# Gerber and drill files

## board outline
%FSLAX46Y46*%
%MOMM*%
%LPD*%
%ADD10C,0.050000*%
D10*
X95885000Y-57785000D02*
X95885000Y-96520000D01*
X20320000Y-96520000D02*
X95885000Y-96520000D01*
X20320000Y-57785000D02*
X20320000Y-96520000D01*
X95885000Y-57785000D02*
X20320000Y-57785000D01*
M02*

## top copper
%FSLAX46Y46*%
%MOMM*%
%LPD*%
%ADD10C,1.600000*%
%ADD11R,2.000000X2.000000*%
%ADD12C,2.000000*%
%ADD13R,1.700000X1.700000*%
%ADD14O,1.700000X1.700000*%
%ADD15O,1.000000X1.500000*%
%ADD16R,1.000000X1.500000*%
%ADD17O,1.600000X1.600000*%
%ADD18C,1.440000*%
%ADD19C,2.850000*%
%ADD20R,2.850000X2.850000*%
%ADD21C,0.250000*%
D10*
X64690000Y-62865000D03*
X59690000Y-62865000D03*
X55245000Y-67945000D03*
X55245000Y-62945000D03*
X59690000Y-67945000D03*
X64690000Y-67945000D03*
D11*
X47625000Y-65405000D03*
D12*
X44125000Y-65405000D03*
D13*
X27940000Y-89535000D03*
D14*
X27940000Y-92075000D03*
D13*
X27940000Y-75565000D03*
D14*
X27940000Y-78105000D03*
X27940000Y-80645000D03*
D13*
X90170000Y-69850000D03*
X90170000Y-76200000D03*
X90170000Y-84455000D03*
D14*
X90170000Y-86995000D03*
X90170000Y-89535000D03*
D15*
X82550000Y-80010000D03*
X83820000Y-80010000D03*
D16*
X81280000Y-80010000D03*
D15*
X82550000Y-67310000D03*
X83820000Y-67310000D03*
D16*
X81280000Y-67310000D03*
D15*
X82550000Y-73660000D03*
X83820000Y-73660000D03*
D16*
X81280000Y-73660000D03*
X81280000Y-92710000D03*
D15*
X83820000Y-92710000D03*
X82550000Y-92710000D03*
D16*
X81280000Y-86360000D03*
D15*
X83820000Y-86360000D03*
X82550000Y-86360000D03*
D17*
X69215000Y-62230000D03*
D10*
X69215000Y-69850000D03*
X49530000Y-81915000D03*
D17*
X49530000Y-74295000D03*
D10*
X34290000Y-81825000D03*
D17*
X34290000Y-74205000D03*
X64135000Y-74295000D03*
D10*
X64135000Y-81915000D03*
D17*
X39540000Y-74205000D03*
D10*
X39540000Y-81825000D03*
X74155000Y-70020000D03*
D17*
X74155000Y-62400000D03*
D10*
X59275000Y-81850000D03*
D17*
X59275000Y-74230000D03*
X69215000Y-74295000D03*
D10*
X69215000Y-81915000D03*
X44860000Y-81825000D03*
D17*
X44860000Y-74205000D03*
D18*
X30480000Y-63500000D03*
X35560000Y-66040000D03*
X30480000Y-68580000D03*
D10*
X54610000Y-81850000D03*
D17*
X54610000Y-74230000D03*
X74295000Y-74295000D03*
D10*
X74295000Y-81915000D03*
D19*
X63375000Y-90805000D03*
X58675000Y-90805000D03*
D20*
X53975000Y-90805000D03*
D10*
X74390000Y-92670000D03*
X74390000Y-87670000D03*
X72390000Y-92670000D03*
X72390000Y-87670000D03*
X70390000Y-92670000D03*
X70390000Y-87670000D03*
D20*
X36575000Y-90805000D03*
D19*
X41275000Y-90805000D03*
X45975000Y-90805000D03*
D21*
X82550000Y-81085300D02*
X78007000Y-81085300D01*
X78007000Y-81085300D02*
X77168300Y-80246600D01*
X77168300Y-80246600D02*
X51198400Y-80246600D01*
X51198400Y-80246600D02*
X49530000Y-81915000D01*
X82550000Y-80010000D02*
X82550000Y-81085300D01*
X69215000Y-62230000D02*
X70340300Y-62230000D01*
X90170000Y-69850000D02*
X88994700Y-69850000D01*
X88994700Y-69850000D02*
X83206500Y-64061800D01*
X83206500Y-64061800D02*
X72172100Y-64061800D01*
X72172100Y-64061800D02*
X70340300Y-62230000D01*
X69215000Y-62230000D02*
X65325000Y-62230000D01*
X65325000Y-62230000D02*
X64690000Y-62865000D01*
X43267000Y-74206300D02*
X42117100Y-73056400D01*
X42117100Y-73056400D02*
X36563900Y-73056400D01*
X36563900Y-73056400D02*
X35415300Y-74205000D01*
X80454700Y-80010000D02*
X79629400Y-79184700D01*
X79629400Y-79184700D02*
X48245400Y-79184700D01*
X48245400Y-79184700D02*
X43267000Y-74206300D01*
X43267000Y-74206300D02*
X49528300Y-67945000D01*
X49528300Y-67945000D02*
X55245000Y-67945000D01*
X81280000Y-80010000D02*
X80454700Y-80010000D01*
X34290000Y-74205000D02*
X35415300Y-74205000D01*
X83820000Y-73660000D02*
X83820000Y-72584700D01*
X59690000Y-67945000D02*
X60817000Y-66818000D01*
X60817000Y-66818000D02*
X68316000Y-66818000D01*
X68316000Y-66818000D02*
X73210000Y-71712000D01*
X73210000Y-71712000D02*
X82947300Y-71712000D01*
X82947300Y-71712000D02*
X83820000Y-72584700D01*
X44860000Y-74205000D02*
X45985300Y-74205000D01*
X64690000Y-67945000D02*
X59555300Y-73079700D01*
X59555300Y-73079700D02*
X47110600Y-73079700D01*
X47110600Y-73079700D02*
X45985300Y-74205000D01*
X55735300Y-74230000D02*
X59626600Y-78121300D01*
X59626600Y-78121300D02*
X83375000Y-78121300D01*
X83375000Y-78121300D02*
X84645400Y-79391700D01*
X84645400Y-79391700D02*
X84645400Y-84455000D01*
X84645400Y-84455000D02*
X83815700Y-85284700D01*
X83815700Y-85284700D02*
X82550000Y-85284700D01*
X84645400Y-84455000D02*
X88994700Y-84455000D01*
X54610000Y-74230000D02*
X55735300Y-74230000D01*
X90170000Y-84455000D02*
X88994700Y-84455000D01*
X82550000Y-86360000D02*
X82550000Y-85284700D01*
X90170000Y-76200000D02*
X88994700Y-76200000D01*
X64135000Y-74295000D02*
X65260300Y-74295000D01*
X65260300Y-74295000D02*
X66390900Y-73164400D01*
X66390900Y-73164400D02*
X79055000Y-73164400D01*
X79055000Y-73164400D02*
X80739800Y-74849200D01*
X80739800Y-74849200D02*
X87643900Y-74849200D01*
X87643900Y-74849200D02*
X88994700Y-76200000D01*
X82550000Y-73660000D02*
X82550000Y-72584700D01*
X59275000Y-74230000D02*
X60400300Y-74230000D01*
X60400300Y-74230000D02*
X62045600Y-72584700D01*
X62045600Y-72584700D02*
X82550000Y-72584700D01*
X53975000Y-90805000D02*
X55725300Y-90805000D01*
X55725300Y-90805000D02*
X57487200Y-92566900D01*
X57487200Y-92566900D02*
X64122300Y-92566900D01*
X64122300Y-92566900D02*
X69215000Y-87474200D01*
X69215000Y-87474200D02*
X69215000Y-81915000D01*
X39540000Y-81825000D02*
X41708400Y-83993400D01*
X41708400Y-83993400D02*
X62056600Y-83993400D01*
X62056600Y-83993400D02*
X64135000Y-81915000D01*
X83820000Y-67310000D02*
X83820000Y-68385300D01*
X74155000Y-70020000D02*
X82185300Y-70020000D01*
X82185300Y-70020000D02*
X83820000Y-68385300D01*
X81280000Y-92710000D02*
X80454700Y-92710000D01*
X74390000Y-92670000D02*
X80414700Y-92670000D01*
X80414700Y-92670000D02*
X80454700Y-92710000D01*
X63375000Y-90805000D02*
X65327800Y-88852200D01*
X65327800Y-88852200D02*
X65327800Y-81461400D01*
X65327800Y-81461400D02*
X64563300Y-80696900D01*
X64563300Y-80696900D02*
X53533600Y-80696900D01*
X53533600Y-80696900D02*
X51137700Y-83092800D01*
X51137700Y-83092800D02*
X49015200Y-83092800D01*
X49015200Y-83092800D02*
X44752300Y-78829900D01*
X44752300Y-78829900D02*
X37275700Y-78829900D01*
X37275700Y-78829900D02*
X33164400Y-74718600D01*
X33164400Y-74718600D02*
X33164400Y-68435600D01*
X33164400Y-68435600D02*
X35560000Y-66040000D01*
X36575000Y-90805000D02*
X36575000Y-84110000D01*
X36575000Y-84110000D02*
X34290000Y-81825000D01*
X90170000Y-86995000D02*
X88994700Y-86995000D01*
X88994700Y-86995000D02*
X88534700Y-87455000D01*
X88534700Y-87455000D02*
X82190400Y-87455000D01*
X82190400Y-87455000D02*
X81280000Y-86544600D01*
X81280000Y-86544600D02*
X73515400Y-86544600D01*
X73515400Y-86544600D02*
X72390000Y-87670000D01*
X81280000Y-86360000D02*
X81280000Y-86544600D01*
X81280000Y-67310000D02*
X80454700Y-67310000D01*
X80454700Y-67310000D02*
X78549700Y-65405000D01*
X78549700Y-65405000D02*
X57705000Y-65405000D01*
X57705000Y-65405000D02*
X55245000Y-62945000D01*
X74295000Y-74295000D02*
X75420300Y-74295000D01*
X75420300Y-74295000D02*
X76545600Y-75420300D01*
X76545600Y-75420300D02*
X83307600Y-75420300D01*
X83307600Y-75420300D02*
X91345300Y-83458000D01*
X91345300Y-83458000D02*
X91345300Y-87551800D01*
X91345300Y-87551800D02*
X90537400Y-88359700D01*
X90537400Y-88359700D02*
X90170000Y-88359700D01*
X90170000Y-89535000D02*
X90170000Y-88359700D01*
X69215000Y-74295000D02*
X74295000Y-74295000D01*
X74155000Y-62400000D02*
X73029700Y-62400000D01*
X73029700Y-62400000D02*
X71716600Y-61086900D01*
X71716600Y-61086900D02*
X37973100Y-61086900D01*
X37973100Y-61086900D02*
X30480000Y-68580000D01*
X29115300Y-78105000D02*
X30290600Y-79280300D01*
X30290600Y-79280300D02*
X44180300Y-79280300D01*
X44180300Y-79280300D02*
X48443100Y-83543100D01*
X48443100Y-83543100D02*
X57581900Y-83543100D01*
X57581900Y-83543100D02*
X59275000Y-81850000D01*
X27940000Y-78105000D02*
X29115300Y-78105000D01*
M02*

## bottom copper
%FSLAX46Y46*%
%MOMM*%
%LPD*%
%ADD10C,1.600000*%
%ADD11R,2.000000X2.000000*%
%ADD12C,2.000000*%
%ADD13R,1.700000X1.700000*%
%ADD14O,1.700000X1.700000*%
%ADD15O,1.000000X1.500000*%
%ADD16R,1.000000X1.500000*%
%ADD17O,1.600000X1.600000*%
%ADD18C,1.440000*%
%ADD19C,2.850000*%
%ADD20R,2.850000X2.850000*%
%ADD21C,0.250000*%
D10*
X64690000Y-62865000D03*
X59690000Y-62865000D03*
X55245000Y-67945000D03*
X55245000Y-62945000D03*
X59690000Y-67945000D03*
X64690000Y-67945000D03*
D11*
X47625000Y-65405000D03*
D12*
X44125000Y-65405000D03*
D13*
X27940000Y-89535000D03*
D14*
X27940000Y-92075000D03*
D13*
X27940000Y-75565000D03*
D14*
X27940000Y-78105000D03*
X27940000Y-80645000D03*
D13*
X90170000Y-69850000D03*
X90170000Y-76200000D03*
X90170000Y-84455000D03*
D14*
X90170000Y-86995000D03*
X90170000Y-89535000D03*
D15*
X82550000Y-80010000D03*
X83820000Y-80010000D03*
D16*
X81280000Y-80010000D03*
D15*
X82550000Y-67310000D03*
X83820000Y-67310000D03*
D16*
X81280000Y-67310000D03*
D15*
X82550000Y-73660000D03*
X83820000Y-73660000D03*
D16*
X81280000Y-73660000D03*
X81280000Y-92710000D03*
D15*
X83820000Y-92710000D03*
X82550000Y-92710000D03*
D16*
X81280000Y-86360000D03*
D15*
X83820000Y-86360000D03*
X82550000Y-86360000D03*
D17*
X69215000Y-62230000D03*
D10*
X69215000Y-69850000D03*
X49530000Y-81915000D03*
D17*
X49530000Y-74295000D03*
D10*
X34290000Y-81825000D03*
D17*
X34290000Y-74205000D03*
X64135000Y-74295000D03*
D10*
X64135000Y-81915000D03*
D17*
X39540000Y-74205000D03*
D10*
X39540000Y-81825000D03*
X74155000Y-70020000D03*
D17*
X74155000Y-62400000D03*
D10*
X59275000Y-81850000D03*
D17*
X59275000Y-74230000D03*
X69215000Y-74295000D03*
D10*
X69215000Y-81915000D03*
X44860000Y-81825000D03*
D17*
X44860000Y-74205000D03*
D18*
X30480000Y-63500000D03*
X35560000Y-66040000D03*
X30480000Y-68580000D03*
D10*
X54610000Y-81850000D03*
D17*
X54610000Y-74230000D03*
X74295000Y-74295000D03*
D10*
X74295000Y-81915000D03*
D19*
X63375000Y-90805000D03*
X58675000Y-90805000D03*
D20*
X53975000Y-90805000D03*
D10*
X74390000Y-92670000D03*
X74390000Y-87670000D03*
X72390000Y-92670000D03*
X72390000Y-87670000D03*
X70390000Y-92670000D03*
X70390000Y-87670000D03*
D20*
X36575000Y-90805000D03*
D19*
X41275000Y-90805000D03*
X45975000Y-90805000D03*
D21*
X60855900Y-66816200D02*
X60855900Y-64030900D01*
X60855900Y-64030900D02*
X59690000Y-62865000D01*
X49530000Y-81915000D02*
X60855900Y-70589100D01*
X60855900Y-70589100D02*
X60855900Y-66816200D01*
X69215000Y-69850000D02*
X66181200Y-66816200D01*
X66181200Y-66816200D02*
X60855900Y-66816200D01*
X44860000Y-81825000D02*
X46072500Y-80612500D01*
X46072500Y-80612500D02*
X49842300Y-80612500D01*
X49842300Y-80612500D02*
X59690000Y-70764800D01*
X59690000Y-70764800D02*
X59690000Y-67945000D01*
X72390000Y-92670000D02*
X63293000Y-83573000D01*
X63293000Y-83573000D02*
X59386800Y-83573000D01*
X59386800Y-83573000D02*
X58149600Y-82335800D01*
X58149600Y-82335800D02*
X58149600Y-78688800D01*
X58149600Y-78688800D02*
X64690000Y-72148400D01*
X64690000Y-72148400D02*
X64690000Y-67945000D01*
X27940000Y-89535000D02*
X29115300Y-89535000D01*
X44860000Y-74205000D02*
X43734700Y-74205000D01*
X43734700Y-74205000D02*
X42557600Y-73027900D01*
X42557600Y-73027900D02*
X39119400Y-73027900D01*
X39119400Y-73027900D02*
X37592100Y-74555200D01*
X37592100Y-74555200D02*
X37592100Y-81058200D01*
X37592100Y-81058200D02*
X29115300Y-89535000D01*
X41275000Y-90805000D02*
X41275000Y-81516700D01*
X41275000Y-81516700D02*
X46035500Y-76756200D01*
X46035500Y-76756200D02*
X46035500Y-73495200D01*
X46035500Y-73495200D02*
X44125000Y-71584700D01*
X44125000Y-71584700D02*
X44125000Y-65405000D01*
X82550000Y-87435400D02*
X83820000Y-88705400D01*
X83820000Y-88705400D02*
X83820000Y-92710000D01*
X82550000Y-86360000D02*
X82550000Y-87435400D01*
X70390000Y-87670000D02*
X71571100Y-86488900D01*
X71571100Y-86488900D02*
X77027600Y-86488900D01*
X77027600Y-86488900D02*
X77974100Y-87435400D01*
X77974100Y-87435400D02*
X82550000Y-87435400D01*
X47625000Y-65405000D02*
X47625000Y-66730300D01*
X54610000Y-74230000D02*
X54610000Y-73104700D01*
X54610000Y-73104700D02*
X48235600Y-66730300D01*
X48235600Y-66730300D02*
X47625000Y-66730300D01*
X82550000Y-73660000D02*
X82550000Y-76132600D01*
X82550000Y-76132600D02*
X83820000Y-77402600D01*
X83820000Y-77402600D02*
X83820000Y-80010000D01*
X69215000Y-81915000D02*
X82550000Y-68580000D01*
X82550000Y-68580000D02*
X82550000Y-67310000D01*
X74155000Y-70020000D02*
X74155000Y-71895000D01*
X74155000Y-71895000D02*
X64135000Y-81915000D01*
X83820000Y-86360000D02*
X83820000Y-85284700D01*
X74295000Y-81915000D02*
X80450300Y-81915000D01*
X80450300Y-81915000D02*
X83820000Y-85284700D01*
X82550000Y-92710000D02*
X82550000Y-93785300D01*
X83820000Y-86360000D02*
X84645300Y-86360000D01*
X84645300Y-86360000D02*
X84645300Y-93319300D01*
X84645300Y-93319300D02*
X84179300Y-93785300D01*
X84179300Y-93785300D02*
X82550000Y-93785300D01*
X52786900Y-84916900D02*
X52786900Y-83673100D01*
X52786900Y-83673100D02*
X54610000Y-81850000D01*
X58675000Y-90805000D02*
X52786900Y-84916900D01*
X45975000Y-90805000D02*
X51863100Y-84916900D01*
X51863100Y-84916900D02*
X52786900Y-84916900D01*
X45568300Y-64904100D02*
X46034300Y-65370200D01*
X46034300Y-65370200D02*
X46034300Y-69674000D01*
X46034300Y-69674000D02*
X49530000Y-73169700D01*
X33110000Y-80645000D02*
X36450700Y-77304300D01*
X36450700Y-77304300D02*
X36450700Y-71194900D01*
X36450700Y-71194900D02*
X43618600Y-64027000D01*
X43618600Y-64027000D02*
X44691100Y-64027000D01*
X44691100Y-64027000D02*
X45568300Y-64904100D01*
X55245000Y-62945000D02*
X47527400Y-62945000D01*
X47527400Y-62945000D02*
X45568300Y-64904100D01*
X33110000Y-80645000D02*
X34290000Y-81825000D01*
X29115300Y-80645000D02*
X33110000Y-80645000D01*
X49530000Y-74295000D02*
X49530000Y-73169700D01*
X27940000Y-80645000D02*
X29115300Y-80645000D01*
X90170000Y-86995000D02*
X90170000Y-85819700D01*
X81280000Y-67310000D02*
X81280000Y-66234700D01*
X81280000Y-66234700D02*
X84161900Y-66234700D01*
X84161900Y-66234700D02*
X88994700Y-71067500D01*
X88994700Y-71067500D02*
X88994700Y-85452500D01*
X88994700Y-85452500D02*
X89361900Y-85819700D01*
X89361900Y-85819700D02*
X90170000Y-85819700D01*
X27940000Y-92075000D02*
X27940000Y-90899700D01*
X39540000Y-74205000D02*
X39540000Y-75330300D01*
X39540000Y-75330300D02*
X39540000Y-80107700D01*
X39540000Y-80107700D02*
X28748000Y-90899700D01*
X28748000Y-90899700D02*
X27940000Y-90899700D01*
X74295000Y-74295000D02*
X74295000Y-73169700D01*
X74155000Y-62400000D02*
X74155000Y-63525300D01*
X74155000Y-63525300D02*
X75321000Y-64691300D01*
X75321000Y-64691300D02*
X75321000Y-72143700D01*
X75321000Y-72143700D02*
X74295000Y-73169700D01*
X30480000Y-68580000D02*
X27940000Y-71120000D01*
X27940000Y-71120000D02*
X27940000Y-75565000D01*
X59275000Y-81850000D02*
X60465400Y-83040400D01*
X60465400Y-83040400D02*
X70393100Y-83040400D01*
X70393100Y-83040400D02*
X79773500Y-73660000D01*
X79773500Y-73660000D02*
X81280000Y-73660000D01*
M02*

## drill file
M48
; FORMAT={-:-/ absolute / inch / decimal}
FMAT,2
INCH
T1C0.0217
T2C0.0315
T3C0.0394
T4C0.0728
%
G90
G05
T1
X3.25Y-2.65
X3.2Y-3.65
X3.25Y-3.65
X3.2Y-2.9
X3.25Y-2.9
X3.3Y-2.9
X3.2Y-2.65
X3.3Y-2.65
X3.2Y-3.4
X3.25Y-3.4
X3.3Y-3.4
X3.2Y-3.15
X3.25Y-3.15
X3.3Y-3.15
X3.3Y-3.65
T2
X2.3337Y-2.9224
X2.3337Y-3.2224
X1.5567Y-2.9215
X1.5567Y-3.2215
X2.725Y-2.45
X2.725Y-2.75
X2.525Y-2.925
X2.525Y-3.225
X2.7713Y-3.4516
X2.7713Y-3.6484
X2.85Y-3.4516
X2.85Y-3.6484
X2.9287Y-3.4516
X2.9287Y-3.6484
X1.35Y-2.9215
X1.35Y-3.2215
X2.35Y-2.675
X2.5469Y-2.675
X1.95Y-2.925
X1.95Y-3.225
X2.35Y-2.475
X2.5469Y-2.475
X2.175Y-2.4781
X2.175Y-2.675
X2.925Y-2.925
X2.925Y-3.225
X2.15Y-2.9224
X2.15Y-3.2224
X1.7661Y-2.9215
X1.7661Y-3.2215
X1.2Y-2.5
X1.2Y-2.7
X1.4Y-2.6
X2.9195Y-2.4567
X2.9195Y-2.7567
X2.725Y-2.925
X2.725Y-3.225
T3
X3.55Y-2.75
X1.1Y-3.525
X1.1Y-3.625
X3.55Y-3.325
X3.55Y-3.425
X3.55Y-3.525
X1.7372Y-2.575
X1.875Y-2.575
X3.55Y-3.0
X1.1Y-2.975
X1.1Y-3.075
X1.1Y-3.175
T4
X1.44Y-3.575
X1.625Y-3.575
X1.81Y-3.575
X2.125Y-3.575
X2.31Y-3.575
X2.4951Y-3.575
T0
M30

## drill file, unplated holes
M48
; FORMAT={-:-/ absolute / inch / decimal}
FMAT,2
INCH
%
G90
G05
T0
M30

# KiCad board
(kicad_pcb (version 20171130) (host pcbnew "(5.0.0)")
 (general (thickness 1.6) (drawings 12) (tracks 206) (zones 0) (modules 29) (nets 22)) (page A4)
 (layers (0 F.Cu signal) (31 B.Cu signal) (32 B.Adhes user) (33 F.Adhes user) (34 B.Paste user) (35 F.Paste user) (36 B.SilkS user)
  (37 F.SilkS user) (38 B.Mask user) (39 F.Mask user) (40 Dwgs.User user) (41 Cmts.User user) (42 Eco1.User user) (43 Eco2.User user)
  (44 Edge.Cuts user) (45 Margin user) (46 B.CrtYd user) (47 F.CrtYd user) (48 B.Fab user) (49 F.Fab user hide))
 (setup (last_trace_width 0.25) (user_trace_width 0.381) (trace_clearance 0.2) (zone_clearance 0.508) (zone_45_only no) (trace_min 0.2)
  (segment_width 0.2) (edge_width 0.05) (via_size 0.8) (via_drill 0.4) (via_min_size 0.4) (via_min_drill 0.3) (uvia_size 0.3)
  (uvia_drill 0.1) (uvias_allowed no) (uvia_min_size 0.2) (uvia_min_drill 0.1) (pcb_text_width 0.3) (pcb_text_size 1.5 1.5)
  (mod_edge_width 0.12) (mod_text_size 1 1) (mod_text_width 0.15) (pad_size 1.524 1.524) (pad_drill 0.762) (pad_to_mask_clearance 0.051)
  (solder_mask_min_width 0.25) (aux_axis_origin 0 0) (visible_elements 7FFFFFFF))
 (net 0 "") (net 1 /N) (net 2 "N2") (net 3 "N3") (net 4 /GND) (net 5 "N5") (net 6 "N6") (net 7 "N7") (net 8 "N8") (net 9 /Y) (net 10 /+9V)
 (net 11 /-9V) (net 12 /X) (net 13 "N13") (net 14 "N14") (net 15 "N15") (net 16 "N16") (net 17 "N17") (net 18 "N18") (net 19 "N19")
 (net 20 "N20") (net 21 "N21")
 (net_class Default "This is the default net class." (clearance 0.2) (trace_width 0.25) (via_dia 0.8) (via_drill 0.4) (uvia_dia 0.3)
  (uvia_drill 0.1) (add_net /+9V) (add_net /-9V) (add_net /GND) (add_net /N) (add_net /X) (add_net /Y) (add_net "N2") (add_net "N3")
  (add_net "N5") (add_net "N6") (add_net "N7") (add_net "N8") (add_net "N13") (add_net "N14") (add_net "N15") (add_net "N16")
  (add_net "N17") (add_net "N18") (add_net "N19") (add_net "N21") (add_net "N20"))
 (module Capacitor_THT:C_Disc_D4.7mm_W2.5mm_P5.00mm (layer F.Cu) (at 59.69 62.865)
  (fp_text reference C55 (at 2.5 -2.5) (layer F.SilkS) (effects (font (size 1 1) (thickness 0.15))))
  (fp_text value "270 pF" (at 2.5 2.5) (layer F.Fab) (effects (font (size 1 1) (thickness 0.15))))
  (pad 2 thru_hole circle (at 5 0) (size 1.6 1.6) (drill 0.8) (layers *.Cu *.Mask) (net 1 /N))
  (pad 1 thru_hole circle (at 0 0) (size 1.6 1.6) (drill 0.8) (layers *.Cu *.Mask) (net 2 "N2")))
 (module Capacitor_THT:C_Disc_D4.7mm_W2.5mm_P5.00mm (layer F.Cu) (at 55.245 67.945 90)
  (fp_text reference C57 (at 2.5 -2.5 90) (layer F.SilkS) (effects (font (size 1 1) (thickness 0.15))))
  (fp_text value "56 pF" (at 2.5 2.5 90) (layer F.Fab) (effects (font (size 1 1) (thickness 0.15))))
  (pad 1 thru_hole circle (at 0 0 90) (size 1.6 1.6) (drill 0.8) (layers *.Cu *.Mask) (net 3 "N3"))
  (pad 2 thru_hole circle (at 5 0 90) (size 1.6 1.6) (drill 0.8) (layers *.Cu *.Mask) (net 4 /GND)))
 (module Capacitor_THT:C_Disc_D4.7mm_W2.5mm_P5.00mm (layer F.Cu) (at 59.69 67.945)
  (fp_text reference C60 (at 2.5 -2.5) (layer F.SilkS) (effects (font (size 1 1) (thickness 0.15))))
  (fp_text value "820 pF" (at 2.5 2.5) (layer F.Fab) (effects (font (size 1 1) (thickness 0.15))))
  (pad 1 thru_hole circle (at 0 0) (size 1.6 1.6) (drill 0.8) (layers *.Cu *.Mask) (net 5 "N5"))
  (pad 2 thru_hole circle (at 5 0) (size 1.6 1.6) (drill 0.8) (layers *.Cu *.Mask) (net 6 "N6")))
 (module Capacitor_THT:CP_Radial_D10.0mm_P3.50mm (layer F.Cu) (at 47.625 65.405 180)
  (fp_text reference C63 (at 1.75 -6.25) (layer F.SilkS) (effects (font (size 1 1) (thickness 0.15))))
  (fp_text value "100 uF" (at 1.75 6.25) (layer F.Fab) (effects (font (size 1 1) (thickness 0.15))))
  (pad 1 thru_hole rect (at 0 0 180) (size 2 2) (drill 1) (layers *.Cu *.Mask) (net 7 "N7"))
  (pad 2 thru_hole circle (at 3.5 0 180) (size 2 2) (drill 1) (layers *.Cu *.Mask) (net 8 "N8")))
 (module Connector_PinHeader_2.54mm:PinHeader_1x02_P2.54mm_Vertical (layer F.Cu) (at 27.94 89.535)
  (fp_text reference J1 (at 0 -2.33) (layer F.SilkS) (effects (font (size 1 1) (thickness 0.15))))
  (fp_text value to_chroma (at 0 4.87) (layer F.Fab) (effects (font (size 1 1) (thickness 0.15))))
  (pad 1 thru_hole rect (at 0 0) (size 1.7 1.7) (drill 1) (layers *.Cu *.Mask) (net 6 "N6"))
  (pad 2 thru_hole oval (at 0 2.54) (size 1.7 1.7) (drill 1) (layers *.Cu *.Mask) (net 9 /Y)))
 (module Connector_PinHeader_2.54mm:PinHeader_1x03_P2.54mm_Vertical (layer F.Cu) (at 27.94 75.565)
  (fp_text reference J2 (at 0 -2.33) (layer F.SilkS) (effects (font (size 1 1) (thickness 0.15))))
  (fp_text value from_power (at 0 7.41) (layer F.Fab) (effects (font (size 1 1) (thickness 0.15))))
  (pad 1 thru_hole rect (at 0 0) (size 1.7 1.7) (drill 1) (layers *.Cu *.Mask) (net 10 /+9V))
  (pad 2 thru_hole oval (at 0 2.54) (size 1.7 1.7) (drill 1) (layers *.Cu *.Mask) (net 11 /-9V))
  (pad 3 thru_hole oval (at 0 5.08) (size 1.7 1.7) (drill 1) (layers *.Cu *.Mask) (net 4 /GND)))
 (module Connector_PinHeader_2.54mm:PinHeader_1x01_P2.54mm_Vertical (layer F.Cu) (at 90.17 69.85)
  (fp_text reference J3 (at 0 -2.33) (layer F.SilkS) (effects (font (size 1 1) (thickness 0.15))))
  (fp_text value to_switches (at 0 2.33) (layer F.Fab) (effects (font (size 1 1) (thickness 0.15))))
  (pad 1 thru_hole rect (at 0 0) (size 1.7 1.7) (drill 1) (layers *.Cu *.Mask) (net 1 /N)))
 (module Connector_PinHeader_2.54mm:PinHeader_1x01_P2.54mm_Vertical (layer F.Cu) (at 90.17 76.2)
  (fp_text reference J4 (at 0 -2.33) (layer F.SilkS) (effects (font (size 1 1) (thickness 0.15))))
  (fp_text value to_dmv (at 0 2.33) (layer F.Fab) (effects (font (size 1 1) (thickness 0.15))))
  (pad 1 thru_hole rect (at 0 0) (size 1.7 1.7) (drill 1) (layers *.Cu *.Mask) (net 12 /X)))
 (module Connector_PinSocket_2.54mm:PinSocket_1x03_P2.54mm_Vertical (layer F.Cu) (at 90.17 84.455)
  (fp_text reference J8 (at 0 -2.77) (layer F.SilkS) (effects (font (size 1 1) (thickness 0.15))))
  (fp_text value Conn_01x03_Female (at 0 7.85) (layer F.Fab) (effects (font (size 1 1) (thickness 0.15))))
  (pad 1 thru_hole rect (at 0 0) (size 1.7 1.7) (drill 1) (layers *.Cu *.Mask) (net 7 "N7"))
  (pad 2 thru_hole oval (at 0 2.54) (size 1.7 1.7) (drill 1) (layers *.Cu *.Mask) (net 4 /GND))
  (pad 3 thru_hole oval (at 0 5.08) (size 1.7 1.7) (drill 1) (layers *.Cu *.Mask) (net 10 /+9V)))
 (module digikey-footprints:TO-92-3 (layer F.Cu) (at 81.28 80.01)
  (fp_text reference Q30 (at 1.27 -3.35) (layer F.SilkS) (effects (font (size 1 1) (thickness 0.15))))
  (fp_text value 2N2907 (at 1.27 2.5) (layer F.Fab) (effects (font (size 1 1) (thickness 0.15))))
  (pad 2 thru_hole oval (at 1.27 0 180) (size 1 1.5) (drill 0.55) (layers *.Cu *.Mask) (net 2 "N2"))
  (pad 3 thru_hole oval (at 2.54 0 180) (size 1 1.5) (drill 0.55) (layers *.Cu *.Mask) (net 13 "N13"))
  (pad 1 thru_hole rect (at 0 0 180) (size 1 1.5) (drill 0.55) (layers *.Cu *.Mask) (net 3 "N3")))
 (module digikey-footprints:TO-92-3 (layer F.Cu) (at 81.28 67.31)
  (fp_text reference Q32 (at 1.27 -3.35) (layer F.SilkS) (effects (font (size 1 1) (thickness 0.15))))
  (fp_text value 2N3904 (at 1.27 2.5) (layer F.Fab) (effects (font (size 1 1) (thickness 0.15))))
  (pad 2 thru_hole oval (at 1.27 0 180) (size 1 1.5) (drill 0.55) (layers *.Cu *.Mask) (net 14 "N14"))
  (pad 3 thru_hole oval (at 2.54 0 180) (size 1 1.5) (drill 0.55) (layers *.Cu *.Mask) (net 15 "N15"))
  (pad 1 thru_hole rect (at 0 0 180) (size 1 1.5) (drill 0.55) (layers *.Cu *.Mask) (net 4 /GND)))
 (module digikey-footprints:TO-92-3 (layer F.Cu) (at 81.28 73.66)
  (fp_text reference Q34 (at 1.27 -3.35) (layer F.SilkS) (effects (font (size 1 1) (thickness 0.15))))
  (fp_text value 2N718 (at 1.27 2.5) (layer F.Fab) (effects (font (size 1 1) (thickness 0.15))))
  (pad 2 thru_hole oval (at 1.27 0 180) (size 1 1.5) (drill 0.55) (layers *.Cu *.Mask) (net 13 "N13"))
  (pad 3 thru_hole oval (at 2.54 0 180) (size 1 1.5) (drill 0.55) (layers *.Cu *.Mask) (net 5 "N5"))
  (pad 1 thru_hole rect (at 0 0 180) (size 1 1.5) (drill 0.55) (layers *.Cu *.Mask) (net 11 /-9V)))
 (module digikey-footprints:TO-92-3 (layer F.Cu) (at 81.28 92.71)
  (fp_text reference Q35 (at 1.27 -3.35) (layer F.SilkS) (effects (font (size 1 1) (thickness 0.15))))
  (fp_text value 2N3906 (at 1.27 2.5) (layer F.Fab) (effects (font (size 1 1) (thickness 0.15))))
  (pad 1 thru_hole rect (at 0 0 180) (size 1 1.5) (drill 0.55) (layers *.Cu *.Mask) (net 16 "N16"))
  (pad 3 thru_hole oval (at 2.54 0 180) (size 1 1.5) (drill 0.55) (layers *.Cu *.Mask) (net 7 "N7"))
  (pad 2 thru_hole oval (at 1.27 0 180) (size 1 1.5) (drill 0.55) (layers *.Cu *.Mask) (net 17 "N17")))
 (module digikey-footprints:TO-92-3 (layer F.Cu) (at 81.28 86.36)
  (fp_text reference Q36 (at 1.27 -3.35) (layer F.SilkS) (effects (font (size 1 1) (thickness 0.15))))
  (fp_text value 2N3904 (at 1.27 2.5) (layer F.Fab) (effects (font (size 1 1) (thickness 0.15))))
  (pad 1 thru_hole rect (at 0 0 180) (size 1 1.5) (drill 0.55) (layers *.Cu *.Mask) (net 4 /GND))
  (pad 3 thru_hole oval (at 2.54 0 180) (size 1 1.5) (drill 0.55) (layers *.Cu *.Mask) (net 17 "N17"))
  (pad 2 thru_hole oval (at 1.27 0 180) (size 1 1.5) (drill 0.55) (layers *.Cu *.Mask) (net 7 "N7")))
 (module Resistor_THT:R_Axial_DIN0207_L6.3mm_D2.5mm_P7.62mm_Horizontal (layer F.Cu) (at 69.215 69.85 90)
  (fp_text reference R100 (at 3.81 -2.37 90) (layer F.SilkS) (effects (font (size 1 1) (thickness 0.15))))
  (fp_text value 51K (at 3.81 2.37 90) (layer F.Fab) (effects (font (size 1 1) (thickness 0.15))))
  (pad 2 thru_hole oval (at 7.62 0 90) (size 1.6 1.6) (drill 0.8) (layers *.Cu *.Mask) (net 1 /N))
  (pad 1 thru_hole circle (at 0 0 90) (size 1.6 1.6) (drill 0.8) (layers *.Cu *.Mask) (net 2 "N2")))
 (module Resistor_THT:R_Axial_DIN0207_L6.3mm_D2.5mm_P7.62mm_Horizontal (layer F.Cu) (at 49.53 81.915 90)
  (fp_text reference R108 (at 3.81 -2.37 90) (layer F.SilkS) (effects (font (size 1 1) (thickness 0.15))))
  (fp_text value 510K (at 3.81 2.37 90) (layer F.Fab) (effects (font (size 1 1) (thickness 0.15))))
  (pad 1 thru_hole circle (at 0 0 90) (size 1.6 1.6) (drill 0.8) (layers *.Cu *.Mask) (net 2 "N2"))
  (pad 2 thru_hole oval (at 7.62 0 90) (size 1.6 1.6) (drill 0.8) (layers *.Cu *.Mask) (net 4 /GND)))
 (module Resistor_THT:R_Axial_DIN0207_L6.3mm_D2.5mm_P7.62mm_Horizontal (layer F.Cu) (at 34.29 81.825 90)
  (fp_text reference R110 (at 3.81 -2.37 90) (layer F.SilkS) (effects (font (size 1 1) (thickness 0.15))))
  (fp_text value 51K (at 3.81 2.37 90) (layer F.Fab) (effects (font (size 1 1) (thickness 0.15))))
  (pad 1 thru_hole circle (at 0 0 90) (size 1.6 1.6) (drill 0.8) (layers *.Cu *.Mask) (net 4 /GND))
  (pad 2 thru_hole oval (at 7.62 0 90) (size 1.6 1.6) (drill 0.8) (layers *.Cu *.Mask) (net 3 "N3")))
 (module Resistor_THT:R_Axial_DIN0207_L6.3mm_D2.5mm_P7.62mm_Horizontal (layer F.Cu) (at 64.135 81.915 90)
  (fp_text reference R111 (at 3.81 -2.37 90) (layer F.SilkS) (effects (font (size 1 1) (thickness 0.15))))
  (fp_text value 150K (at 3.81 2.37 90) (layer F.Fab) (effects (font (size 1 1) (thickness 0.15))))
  (pad 2 thru_hole oval (at 7.62 0 90) (size 1.6 1.6) (drill 0.8) (layers *.Cu *.Mask) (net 12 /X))
  (pad 1 thru_hole circle (at 0 0 90) (size 1.6 1.6) (drill 0.8) (layers *.Cu *.Mask) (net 15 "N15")))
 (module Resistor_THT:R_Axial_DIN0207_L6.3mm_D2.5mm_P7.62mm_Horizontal (layer F.Cu) (at 39.54 81.825 90)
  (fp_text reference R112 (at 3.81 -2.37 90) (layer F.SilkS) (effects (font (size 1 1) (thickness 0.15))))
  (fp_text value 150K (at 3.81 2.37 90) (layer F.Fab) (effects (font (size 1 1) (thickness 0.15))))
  (pad 2 thru_hole oval (at 7.62 0 90) (size 1.6 1.6) (drill 0.8) (layers *.Cu *.Mask) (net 9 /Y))
  (pad 1 thru_hole circle (at 0 0 90) (size 1.6 1.6) (drill 0.8) (layers *.Cu *.Mask) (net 15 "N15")))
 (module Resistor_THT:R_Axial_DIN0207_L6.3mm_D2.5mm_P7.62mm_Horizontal (layer F.Cu) (at 74.155 70.02 90)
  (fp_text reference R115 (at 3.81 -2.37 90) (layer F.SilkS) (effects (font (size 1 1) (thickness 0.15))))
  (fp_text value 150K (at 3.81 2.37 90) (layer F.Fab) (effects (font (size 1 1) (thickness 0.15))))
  (pad 1 thru_hole circle (at 0 0 90) (size 1.6 1.6) (drill 0.8) (layers *.Cu *.Mask) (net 15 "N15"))
  (pad 2 thru_hole oval (at 7.62 0 90) (size 1.6 1.6) (drill 0.8) (layers *.Cu *.Mask) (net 10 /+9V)))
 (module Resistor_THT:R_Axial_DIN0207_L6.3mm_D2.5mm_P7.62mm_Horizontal (layer F.Cu) (at 59.275 81.85 90)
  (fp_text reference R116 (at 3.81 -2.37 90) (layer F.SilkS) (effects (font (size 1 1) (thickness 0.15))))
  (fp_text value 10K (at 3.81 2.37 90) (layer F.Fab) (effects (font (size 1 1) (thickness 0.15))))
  (pad 1 thru_hole circle (at 0 0 90) (size 1.6 1.6) (drill 0.8) (layers *.Cu *.Mask) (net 11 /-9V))
  (pad 2 thru_hole oval (at 7.62 0 90) (size 1.6 1.6) (drill 0.8) (layers *.Cu *.Mask) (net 13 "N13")))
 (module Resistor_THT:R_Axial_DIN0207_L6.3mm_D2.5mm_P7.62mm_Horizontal (layer F.Cu) (at 69.215 81.915 90)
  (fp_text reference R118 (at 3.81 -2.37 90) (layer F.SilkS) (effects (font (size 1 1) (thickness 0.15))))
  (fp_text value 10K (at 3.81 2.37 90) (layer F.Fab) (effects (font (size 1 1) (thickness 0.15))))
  (pad 2 thru_hole oval (at 7.62 0 90) (size 1.6 1.6) (drill 0.8) (layers *.Cu *.Mask) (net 10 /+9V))
  (pad 1 thru_hole circle (at 0 0 90) (size 1.6 1.6) (drill 0.8) (layers *.Cu *.Mask) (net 14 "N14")))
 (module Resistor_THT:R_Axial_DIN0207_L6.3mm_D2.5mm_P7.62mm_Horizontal (layer F.Cu) (at 44.86 81.825 90)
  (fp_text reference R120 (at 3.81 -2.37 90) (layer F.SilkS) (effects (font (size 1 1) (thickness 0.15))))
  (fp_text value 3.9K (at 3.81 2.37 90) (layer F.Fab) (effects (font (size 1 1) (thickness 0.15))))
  (pad 1 thru_hole circle (at 0 0 90) (size 1.6 1.6) (drill 0.8) (layers *.Cu *.Mask) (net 5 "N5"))
  (pad 2 thru_hole oval (at 7.62 0 90) (size 1.6 1.6) (drill 0.8) (layers *.Cu *.Mask) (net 6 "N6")))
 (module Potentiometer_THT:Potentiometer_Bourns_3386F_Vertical (layer F.Cu) (at 30.48 68.58)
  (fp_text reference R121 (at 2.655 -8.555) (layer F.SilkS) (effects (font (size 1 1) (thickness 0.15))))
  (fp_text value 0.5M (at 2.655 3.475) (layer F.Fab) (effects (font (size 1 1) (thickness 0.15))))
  (pad 3 thru_hole circle (at 0 -5.08) (size 1.44 1.44) (drill 0.8) (layers *.Cu *.Mask))
  (pad 2 thru_hole circle (at 5.08 -2.54) (size 1.44 1.44) (drill 0.8) (layers *.Cu *.Mask) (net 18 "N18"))
  (pad 1 thru_hole circle (at 0 0) (size 1.44 1.44) (drill 0.8) (layers *.Cu *.Mask) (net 10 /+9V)))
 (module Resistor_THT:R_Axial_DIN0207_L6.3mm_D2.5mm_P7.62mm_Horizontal (layer F.Cu) (at 54.61 81.85 90)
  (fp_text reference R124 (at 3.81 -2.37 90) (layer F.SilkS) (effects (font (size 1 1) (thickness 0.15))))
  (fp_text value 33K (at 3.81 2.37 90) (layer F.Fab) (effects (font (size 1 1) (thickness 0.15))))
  (pad 1 thru_hole circle (at 0 0 90) (size 1.6 1.6) (drill 0.8) (layers *.Cu *.Mask) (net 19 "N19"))
  (pad 2 thru_hole oval (at 7.62 0 90) (size 1.6 1.6) (drill 0.8) (layers *.Cu *.Mask) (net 7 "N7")))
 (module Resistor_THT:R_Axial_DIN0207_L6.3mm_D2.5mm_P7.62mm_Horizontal (layer F.Cu) (at 74.295 81.915 90)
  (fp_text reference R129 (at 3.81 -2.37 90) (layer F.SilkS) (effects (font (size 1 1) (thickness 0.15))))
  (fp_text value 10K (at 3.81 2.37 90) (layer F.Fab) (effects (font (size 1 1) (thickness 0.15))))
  (pad 2 thru_hole oval (at 7.62 0 90) (size 1.6 1.6) (drill 0.8) (layers *.Cu *.Mask) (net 10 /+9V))
  (pad 1 thru_hole circle (at 0 0 90) (size 1.6 1.6) (drill 0.8) (layers *.Cu *.Mask) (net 17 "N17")))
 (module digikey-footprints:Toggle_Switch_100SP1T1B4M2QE (layer F.Cu) (at 53.975 90.805)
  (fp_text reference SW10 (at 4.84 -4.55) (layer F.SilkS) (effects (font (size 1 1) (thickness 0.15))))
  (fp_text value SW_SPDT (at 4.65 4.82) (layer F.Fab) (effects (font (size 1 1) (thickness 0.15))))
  (pad 3 thru_hole circle (at 9.4 0) (size 2.85 2.85) (drill 1.85) (layers *.Cu *.Mask) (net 18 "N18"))
  (pad 2 thru_hole circle (at 4.7 0) (size 2.85 2.85) (drill 1.85) (layers *.Cu *.Mask) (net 19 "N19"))
  (pad 1 thru_hole rect (at 0 0) (size 2.85 2.85) (drill 1.85) (layers *.Cu *.Mask) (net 14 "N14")))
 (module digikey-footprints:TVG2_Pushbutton (layer F.Cu) (at 72.39 90.17 180)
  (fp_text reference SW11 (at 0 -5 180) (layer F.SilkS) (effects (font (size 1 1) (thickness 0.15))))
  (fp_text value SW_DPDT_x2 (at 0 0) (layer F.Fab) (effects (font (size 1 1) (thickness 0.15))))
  (pad 1 thru_hole circle (at -2 -2.5 180) (size 1.6 1.6) (drill 0.8) (layers *.Cu *.Mask) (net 16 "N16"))
  (pad 4 thru_hole circle (at -2 2.5 180) (size 1.6 1.6) (drill 0.8) (layers *.Cu *.Mask) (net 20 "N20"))
  (pad 2 thru_hole circle (at 0 -2.5 180) (size 1.6 1.6) (drill 0.8) (layers *.Cu *.Mask) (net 6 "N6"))
  (pad 5 thru_hole circle (at 0 2.5 180) (size 1.6 1.6) (drill 0.8) (layers *.Cu *.Mask) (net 4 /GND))
  (pad 3 thru_hole circle (at 2 -2.5 180) (size 1.6 1.6) (drill 0.8) (layers *.Cu *.Mask) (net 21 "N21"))
  (pad 6 thru_hole circle (at 2 2.5 180) (size 1.6 1.6) (drill 0.8) (layers *.Cu *.Mask) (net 7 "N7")))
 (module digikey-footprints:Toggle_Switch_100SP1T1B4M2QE (layer F.Cu) (at 36.575 90.805)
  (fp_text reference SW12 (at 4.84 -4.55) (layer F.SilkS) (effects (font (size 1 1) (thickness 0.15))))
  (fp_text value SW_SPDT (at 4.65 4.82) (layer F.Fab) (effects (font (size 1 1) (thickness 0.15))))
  (pad 1 thru_hole rect (at 0 0) (size 2.85 2.85) (drill 1.85) (layers *.Cu *.Mask) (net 4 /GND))
  (pad 2 thru_hole circle (at 4.7 0) (size 2.85 2.85) (drill 1.85) (layers *.Cu *.Mask) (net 8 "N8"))
  (pad 3 thru_hole circle (at 9.4 0) (size 2.85 2.85) (drill 1.85) (layers *.Cu *.Mask) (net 19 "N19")))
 (gr_line (start 95.885 57.785) (end 95.885 96.52) (layer Edge.Cuts) (width 0.05))
 (gr_line (start 20.32 96.52) (end 95.885 96.52) (layer Edge.Cuts) (width 0.05))
 (gr_line (start 20.32 57.785) (end 20.32 96.52) (layer Edge.Cuts) (width 0.05))
 (gr_line (start 95.885 57.785) (end 20.32 57.785) (layer Edge.Cuts) (width 0.05))
 (segment (start 60.8559 66.8162) (end 60.8559 64.0309) (width 0.25) (layer B.Cu) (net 2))
 (segment (start 60.8559 64.0309) (end 59.69 62.865) (width 0.25) (layer B.Cu) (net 2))
 (segment (start 49.53 81.915) (end 60.8559 70.5891) (width 0.25) (layer B.Cu) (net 2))
 (segment (start 60.8559 70.5891) (end 60.8559 66.8162) (width 0.25) (layer B.Cu) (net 2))
 (segment (start 69.215 69.85) (end 66.1812 66.8162) (width 0.25) (layer B.Cu) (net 2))
 (segment (start 66.1812 66.8162) (end 60.8559 66.8162) (width 0.25) (layer B.Cu) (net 2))
 (segment (start 82.55 81.0853) (end 78.007 81.0853) (width 0.25) (layer F.Cu) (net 2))
 (segment (start 78.007 81.0853) (end 77.1683 80.2466) (width 0.25) (layer F.Cu) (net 2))
 (segment (start 77.1683 80.2466) (end 51.1984 80.2466) (width 0.25) (layer F.Cu) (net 2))
 (segment (start 51.1984 80.2466) (end 49.53 81.915) (width 0.25) (layer F.Cu) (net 2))
 (segment (start 82.55 80.01) (end 82.55 81.0853) (width 0.25) (layer F.Cu) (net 2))
 (segment (start 69.215 62.23) (end 70.3403 62.23) (width 0.25) (layer F.Cu) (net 1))
 (segment (start 90.17 69.85) (end 88.9947 69.85) (width 0.25) (layer F.Cu) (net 1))
 (segment (start 88.9947 69.85) (end 83.2065 64.0618) (width 0.25) (layer F.Cu) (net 1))
 (segment (start 83.2065 64.0618) (end 72.1721 64.0618) (width 0.25) (layer F.Cu) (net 1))
 (segment (start 72.1721 64.0618) (end 70.3403 62.23) (width 0.25) (layer F.Cu) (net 1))
 (segment (start 69.215 62.23) (end 65.325 62.23) (width 0.25) (layer F.Cu) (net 1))
 (segment (start 65.325 62.23) (end 64.69 62.865) (width 0.25) (layer F.Cu) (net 1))
 (segment (start 43.267 74.2063) (end 42.1171 73.0564) (width 0.25) (layer F.Cu) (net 3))
 (segment (start 42.1171 73.0564) (end 36.5639 73.0564) (width 0.25) (layer F.Cu) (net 3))
 (segment (start 36.5639 73.0564) (end 35.4153 74.205) (width 0.25) (layer F.Cu) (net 3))
 (segment (start 80.4547 80.01) (end 79.6294 79.1847) (width 0.25) (layer F.Cu) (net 3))
 (segment (start 79.6294 79.1847) (end 48.2454 79.1847) (width 0.25) (layer F.Cu) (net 3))
 (segment (start 48.2454 79.1847) (end 43.267 74.2063) (width 0.25) (layer F.Cu) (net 3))
 (segment (start 43.267 74.2063) (end 49.5283 67.945) (width 0.25) (layer F.Cu) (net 3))
 (segment (start 49.5283 67.945) (end 55.245 67.945) (width 0.25) (layer F.Cu) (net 3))
 (segment (start 81.28 80.01) (end 80.4547 80.01) (width 0.25) (layer F.Cu) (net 3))
 (segment (start 34.29 74.205) (end 35.4153 74.205) (width 0.25) (layer F.Cu) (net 3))
 (segment (start 44.86 81.825) (end 46.0725 80.6125) (width 0.25) (layer B.Cu) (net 5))
 (segment (start 46.0725 80.6125) (end 49.8423 80.6125) (width 0.25) (layer B.Cu) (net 5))
 (segment (start 49.8423 80.6125) (end 59.69 70.7648) (width 0.25) (layer B.Cu) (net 5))
 (segment (start 59.69 70.7648) (end 59.69 67.945) (width 0.25) (layer B.Cu) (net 5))
 (segment (start 83.82 73.66) (end 83.82 72.5847) (width 0.25) (layer F.Cu) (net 5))
 (segment (start 59.69 67.945) (end 60.817 66.818) (width 0.25) (layer F.Cu) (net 5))
 (segment (start 60.817 66.818) (end 68.316 66.818) (width 0.25) (layer F.Cu) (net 5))
 (segment (start 68.316 66.818) (end 73.21 71.712) (width 0.25) (layer F.Cu) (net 5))
 (segment (start 73.21 71.712) (end 82.9473 71.712) (width 0.25) (layer F.Cu) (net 5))
 (segment (start 82.9473 71.712) (end 83.82 72.5847) (width 0.25) (layer F.Cu) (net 5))
 (segment (start 72.39 92.67) (end 63.293 83.573) (width 0.25) (layer B.Cu) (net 6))
 (segment (start 63.293 83.573) (end 59.3868 83.573) (width 0.25) (layer B.Cu) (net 6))
 (segment (start 59.3868 83.573) (end 58.1496 82.3358) (width 0.25) (layer B.Cu) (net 6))
 (segment (start 58.1496 82.3358) (end 58.1496 78.6888) (width 0.25) (layer B.Cu) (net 6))
 (segment (start 58.1496 78.6888) (end 64.69 72.1484) (width 0.25) (layer B.Cu) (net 6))
 (segment (start 64.69 72.1484) (end 64.69 67.945) (width 0.25) (layer B.Cu) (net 6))
 (segment (start 44.86 74.205) (end 45.9853 74.205) (width 0.25) (layer F.Cu) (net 6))
 (segment (start 64.69 67.945) (end 59.5553 73.0797) (width 0.25) (layer F.Cu) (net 6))
 (segment (start 59.5553 73.0797) (end 47.1106 73.0797) (width 0.25) (layer F.Cu) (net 6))
 (segment (start 47.1106 73.0797) (end 45.9853 74.205) (width 0.25) (layer F.Cu) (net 6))
 (segment (start 27.94 89.535) (end 29.1153 89.535) (width 0.25) (layer B.Cu) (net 6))
 (segment (start 44.86 74.205) (end 43.7347 74.205) (width 0.25) (layer B.Cu) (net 6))
 (segment (start 43.7347 74.205) (end 42.5576 73.0279) (width 0.25) (layer B.Cu) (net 6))
 (segment (start 42.5576 73.0279) (end 39.1194 73.0279) (width 0.25) (layer B.Cu) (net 6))
 (segment (start 39.1194 73.0279) (end 37.5921 74.5552) (width 0.25) (layer B.Cu) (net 6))
 (segment (start 37.5921 74.5552) (end 37.5921 81.0582) (width 0.25) (layer B.Cu) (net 6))
 (segment (start 37.5921 81.0582) (end 29.1153 89.535) (width 0.25) (layer B.Cu) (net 6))
 (segment (start 41.275 90.805) (end 41.275 81.5167) (width 0.25) (layer B.Cu) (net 8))
 (segment (start 41.275 81.5167) (end 46.0355 76.7562) (width 0.25) (layer B.Cu) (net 8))
 (segment (start 46.0355 76.7562) (end 46.0355 73.4952) (width 0.25) (layer B.Cu) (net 8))
 (segment (start 46.0355 73.4952) (end 44.125 71.5847) (width 0.25) (layer B.Cu) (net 8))
 (segment (start 44.125 71.5847) (end 44.125 65.405) (width 0.25) (layer B.Cu) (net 8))
 (segment (start 55.7353 74.23) (end 59.6266 78.1213) (width 0.25) (layer F.Cu) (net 7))
 (segment (start 59.6266 78.1213) (end 83.375 78.1213) (width 0.25) (layer F.Cu) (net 7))
 (segment (start 83.375 78.1213) (end 84.6454 79.3917) (width 0.25) (layer F.Cu) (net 7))
 (segment (start 84.6454 79.3917) (end 84.6454 84.455) (width 0.25) (layer F.Cu) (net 7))
 (segment (start 84.6454 84.455) (end 83.8157 85.2847) (width 0.25) (layer F.Cu) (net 7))
 (segment (start 83.8157 85.2847) (end 82.55 85.2847) (width 0.25) (layer F.Cu) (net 7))
 (segment (start 84.6454 84.455) (end 88.9947 84.455) (width 0.25) (layer F.Cu) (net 7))
 (segment (start 54.61 74.23) (end 55.7353 74.23) (width 0.25) (layer F.Cu) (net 7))
 (segment (start 90.17 84.455) (end 88.9947 84.455) (width 0.25) (layer F.Cu) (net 7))
 (segment (start 82.55 86.36) (end 82.55 85.2847) (width 0.25) (layer F.Cu) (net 7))
 (segment (start 82.55 87.4354) (end 83.82 88.7054) (width 0.25) (layer B.Cu) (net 7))
 (segment (start 83.82 88.7054) (end 83.82 92.71) (width 0.25) (layer B.Cu) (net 7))
 (segment (start 82.55 86.36) (end 82.55 87.4354) (width 0.25) (layer B.Cu) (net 7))
 (segment (start 70.39 87.67) (end 71.5711 86.4889) (width 0.25) (layer B.Cu) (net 7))
 (segment (start 71.5711 86.4889) (end 77.0276 86.4889) (width 0.25) (layer B.Cu) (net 7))
 (segment (start 77.0276 86.4889) (end 77.9741 87.4354) (width 0.25) (layer B.Cu) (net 7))
 (segment (start 77.9741 87.4354) (end 82.55 87.4354) (width 0.25) (layer B.Cu) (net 7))
 (segment (start 47.625 65.405) (end 47.625 66.7303) (width 0.25) (layer B.Cu) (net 7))
 (segment (start 54.61 74.23) (end 54.61 73.1047) (width 0.25) (layer B.Cu) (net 7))
 (segment (start 54.61 73.1047) (end 48.2356 66.7303) (width 0.25) (layer B.Cu) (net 7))
 (segment (start 48.2356 66.7303) (end 47.625 66.7303) (width 0.25) (layer B.Cu) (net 7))
 (segment (start 90.17 76.2) (end 88.9947 76.2) (width 0.25) (layer F.Cu) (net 12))
 (segment (start 64.135 74.295) (end 65.2603 74.295) (width 0.25) (layer F.Cu) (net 12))
 (segment (start 65.2603 74.295) (end 66.3909 73.1644) (width 0.25) (layer F.Cu) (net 12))
 (segment (start 66.3909 73.1644) (end 79.055 73.1644) (width 0.25) (layer F.Cu) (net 12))
 (segment (start 79.055 73.1644) (end 80.7398 74.8492) (width 0.25) (layer F.Cu) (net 12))
 (segment (start 80.7398 74.8492) (end 87.6439 74.8492) (width 0.25) (layer F.Cu) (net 12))
 (segment (start 87.6439 74.8492) (end 88.9947 76.2) (width 0.25) (layer F.Cu) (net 12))
 (segment (start 82.55 73.66) (end 82.55 72.5847) (width 0.25) (layer F.Cu) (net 13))
 (segment (start 59.275 74.23) (end 60.4003 74.23) (width 0.25) (layer F.Cu) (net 13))
 (segment (start 60.4003 74.23) (end 62.0456 72.5847) (width 0.25) (layer F.Cu) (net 13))
 (segment (start 62.0456 72.5847) (end 82.55 72.5847) (width 0.25) (layer F.Cu) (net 13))
 (segment (start 82.55 73.66) (end 82.55 76.1326) (width 0.25) (layer B.Cu) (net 13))
 (segment (start 82.55 76.1326) (end 83.82 77.4026) (width 0.25) (layer B.Cu) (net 13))
 (segment (start 83.82 77.4026) (end 83.82 80.01) (width 0.25) (layer B.Cu) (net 13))
 (segment (start 53.975 90.805) (end 55.7253 90.805) (width 0.25) (layer F.Cu) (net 14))
 (segment (start 55.7253 90.805) (end 57.4872 92.5669) (width 0.25) (layer F.Cu) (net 14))
 (segment (start 57.4872 92.5669) (end 64.1223 92.5669) (width 0.25) (layer F.Cu) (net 14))
 (segment (start 64.1223 92.5669) (end 69.215 87.4742) (width 0.25) (layer F.Cu) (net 14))
 (segment (start 69.215 87.4742) (end 69.215 81.915) (width 0.25) (layer F.Cu) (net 14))
 (segment (start 69.215 81.915) (end 82.55 68.58) (width 0.25) (layer B.Cu) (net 14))
 (segment (start 82.55 68.58) (end 82.55 67.31) (width 0.25) (layer B.Cu) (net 14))
 (segment (start 74.155 70.02) (end 74.155 71.895) (width 0.25) (layer B.Cu) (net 15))
 (segment (start 74.155 71.895) (end 64.135 81.915) (width 0.25) (layer B.Cu) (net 15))
 (segment (start 39.54 81.825) (end 41.7084 83.9934) (width 0.25) (layer F.Cu) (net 15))
 (segment (start 41.7084 83.9934) (end 62.0566 83.9934) (width 0.25) (layer F.Cu) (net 15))
 (segment (start 62.0566 83.9934) (end 64.135 81.915) (width 0.25) (layer F.Cu) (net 15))
 (segment (start 83.82 67.31) (end 83.82 68.3853) (width 0.25) (layer F.Cu) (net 15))
 (segment (start 74.155 70.02) (end 82.1853 70.02) (width 0.25) (layer F.Cu) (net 15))
 (segment (start 82.1853 70.02) (end 83.82 68.3853) (width 0.25) (layer F.Cu) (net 15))
 (segment (start 83.82 86.36) (end 83.82 85.2847) (width 0.25) (layer B.Cu) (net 17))
 (segment (start 74.295 81.915) (end 80.4503 81.915) (width 0.25) (layer B.Cu) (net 17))
 (segment (start 80.4503 81.915) (end 83.82 85.2847) (width 0.25) (layer B.Cu) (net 17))
 (segment (start 82.55 92.71) (end 82.55 93.7853) (width 0.25) (layer B.Cu) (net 17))
 (segment (start 83.82 86.36) (end 84.6453 86.36) (width 0.25) (layer B.Cu) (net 17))
 (segment (start 84.6453 86.36) (end 84.6453 93.3193) (width 0.25) (layer B.Cu) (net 17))
 (segment (start 84.6453 93.3193) (end 84.1793 93.7853) (width 0.25) (layer B.Cu) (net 17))
 (segment (start 84.1793 93.7853) (end 82.55 93.7853) (width 0.25) (layer B.Cu) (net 17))
 (segment (start 81.28 92.71) (end 80.4547 92.71) (width 0.25) (layer F.Cu) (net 16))
 (segment (start 74.39 92.67) (end 80.4147 92.67) (width 0.25) (layer F.Cu) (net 16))
 (segment (start 80.4147 92.67) (end 80.4547 92.71) (width 0.25) (layer F.Cu) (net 16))
 (segment (start 63.375 90.805) (end 65.3278 88.8522) (width 0.25) (layer F.Cu) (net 18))
 (segment (start 65.3278 88.8522) (end 65.3278 81.4614) (width 0.25) (layer F.Cu) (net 18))
 (segment (start 65.3278 81.4614) (end 64.5633 80.6969) (width 0.25) (layer F.Cu) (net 18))
 (segment (start 64.5633 80.6969) (end 53.5336 80.6969) (width 0.25) (layer F.Cu) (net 18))
 (segment (start 53.5336 80.6969) (end 51.1377 83.0928) (width 0.25) (layer F.Cu) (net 18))
 (segment (start 51.1377 83.0928) (end 49.0152 83.0928) (width 0.25) (layer F.Cu) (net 18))
 (segment (start 49.0152 83.0928) (end 44.7523 78.8299) (width 0.25) (layer F.Cu) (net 18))
 (segment (start 44.7523 78.8299) (end 37.2757 78.8299) (width 0.25) (layer F.Cu) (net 18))
 (segment (start 37.2757 78.8299) (end 33.1644 74.7186) (width 0.25) (layer F.Cu) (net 18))
 (segment (start 33.1644 74.7186) (end 33.1644 68.4356) (width 0.25) (layer F.Cu) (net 18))
 (segment (start 33.1644 68.4356) (end 35.56 66.04) (width 0.25) (layer F.Cu) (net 18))
 (segment (start 52.7869 84.9169) (end 52.7869 83.6731) (width 0.25) (layer B.Cu) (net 19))
 (segment (start 52.7869 83.6731) (end 54.61 81.85) (width 0.25) (layer B.Cu) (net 19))
 (segment (start 58.675 90.805) (end 52.7869 84.9169) (width 0.25) (layer B.Cu) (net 19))
 (segment (start 45.975 90.805) (end 51.8631 84.9169) (width 0.25) (layer B.Cu) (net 19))
 (segment (start 51.8631 84.9169) (end 52.7869 84.9169) (width 0.25) (layer B.Cu) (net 19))
 (segment (start 36.575 90.805) (end 36.575 84.11) (width 0.25) (layer F.Cu) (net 4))
 (segment (start 36.575 84.11) (end 34.29 81.825) (width 0.25) (layer F.Cu) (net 4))
 (segment (start 45.5683 64.9041) (end 46.0343 65.3702) (width 0.25) (layer B.Cu) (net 4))
 (segment (start 46.0343 65.3702) (end 46.0343 69.674) (width 0.25) (layer B.Cu) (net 4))
 (segment (start 46.0343 69.674) (end 49.53 73.1697) (width 0.25) (layer B.Cu) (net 4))
 (segment (start 33.11 80.645) (end 36.4507 77.3043) (width 0.25) (layer B.Cu) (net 4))
 (segment (start 36.4507 77.3043) (end 36.4507 71.1949) (width 0.25) (layer B.Cu) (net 4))
 (segment (start 36.4507 71.1949) (end 43.6186 64.027) (width 0.25) (layer B.Cu) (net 4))
 (segment (start 43.6186 64.027) (end 44.6911 64.027) (width 0.25) (layer B.Cu) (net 4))
 (segment (start 44.6911 64.027) (end 45.5683 64.9041) (width 0.25) (layer B.Cu) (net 4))
 (segment (start 55.245 62.945) (end 47.5274 62.945) (width 0.25) (layer B.Cu) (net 4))
 (segment (start 47.5274 62.945) (end 45.5683 64.9041) (width 0.25) (layer B.Cu) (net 4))
 (segment (start 33.11 80.645) (end 34.29 81.825) (width 0.25) (layer B.Cu) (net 4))
 (segment (start 29.1153 80.645) (end 33.11 80.645) (width 0.25) (layer B.Cu) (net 4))
 (segment (start 49.53 74.295) (end 49.53 73.1697) (width 0.25) (layer B.Cu) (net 4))
 (segment (start 27.94 80.645) (end 29.1153 80.645) (width 0.25) (layer B.Cu) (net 4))
 (segment (start 90.17 86.995) (end 90.17 85.8197) (width 0.25) (layer B.Cu) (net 4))
 (segment (start 81.28 67.31) (end 81.28 66.2347) (width 0.25) (layer B.Cu) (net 4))
 (segment (start 81.28 66.2347) (end 84.1619 66.2347) (width 0.25) (layer B.Cu) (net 4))
 (segment (start 84.1619 66.2347) (end 88.9947 71.0675) (width 0.25) (layer B.Cu) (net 4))
 (segment (start 88.9947 71.0675) (end 88.9947 85.4525) (width 0.25) (layer B.Cu) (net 4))
 (segment (start 88.9947 85.4525) (end 89.3619 85.8197) (width 0.25) (layer B.Cu) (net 4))
 (segment (start 89.3619 85.8197) (end 90.17 85.8197) (width 0.25) (layer B.Cu) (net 4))
 (segment (start 90.17 86.995) (end 88.9947 86.995) (width 0.25) (layer F.Cu) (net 4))
 (segment (start 88.9947 86.995) (end 88.5347 87.455) (width 0.25) (layer F.Cu) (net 4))
 (segment (start 88.5347 87.455) (end 82.1904 87.455) (width 0.25) (layer F.Cu) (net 4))
 (segment (start 82.1904 87.455) (end 81.28 86.5446) (width 0.25) (layer F.Cu) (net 4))
 (segment (start 81.28 86.5446) (end 73.5154 86.5446) (width 0.25) (layer F.Cu) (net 4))
 (segment (start 73.5154 86.5446) (end 72.39 87.67) (width 0.25) (layer F.Cu) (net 4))
 (segment (start 81.28 86.36) (end 81.28 86.5446) (width 0.25) (layer F.Cu) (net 4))
 (segment (start 81.28 67.31) (end 80.4547 67.31) (width 0.25) (layer F.Cu) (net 4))
 (segment (start 80.4547 67.31) (end 78.5497 65.405) (width 0.25) (layer F.Cu) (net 4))
 (segment (start 78.5497 65.405) (end 57.705 65.405) (width 0.25) (layer F.Cu) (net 4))
 (segment (start 57.705 65.405) (end 55.245 62.945) (width 0.25) (layer F.Cu) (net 4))
 (segment (start 27.94 92.075) (end 27.94 90.8997) (width 0.25) (layer B.Cu) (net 9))
 (segment (start 39.54 74.205) (end 39.54 75.3303) (width 0.25) (layer B.Cu) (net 9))
 (segment (start 39.54 75.3303) (end 39.54 80.1077) (width 0.25) (layer B.Cu) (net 9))
 (segment (start 39.54 80.1077) (end 28.748 90.8997) (width 0.25) (layer B.Cu) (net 9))
 (segment (start 28.748 90.8997) (end 27.94 90.8997) (width 0.25) (layer B.Cu) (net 9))
 (segment (start 74.295 74.295) (end 75.4203 74.295) (width 0.25) (layer F.Cu) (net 10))
 (segment (start 75.4203 74.295) (end 76.5456 75.4203) (width 0.25) (layer F.Cu) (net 10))
 (segment (start 76.5456 75.4203) (end 83.3076 75.4203) (width 0.25) (layer F.Cu) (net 10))
 (segment (start 83.3076 75.4203) (end 91.3453 83.458) (width 0.25) (layer F.Cu) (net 10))
 (segment (start 91.3453 83.458) (end 91.3453 87.5518) (width 0.25) (layer F.Cu) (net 10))
 (segment (start 91.3453 87.5518) (end 90.5374 88.3597) (width 0.25) (layer F.Cu) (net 10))
 (segment (start 90.5374 88.3597) (end 90.17 88.3597) (width 0.25) (layer F.Cu) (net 10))
 (segment (start 90.17 89.535) (end 90.17 88.3597) (width 0.25) (layer F.Cu) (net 10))
 (segment (start 69.215 74.295) (end 74.295 74.295) (width 0.25) (layer F.Cu) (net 10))
 (segment (start 74.295 74.295) (end 74.295 73.1697) (width 0.25) (layer B.Cu) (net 10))
 (segment (start 74.155 62.4) (end 74.155 63.5253) (width 0.25) (layer B.Cu) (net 10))
 (segment (start 74.155 63.5253) (end 75.321 64.6913) (width 0.25) (layer B.Cu) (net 10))
 (segment (start 75.321 64.6913) (end 75.321 72.1437) (width 0.25) (layer B.Cu) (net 10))
 (segment (start 75.321 72.1437) (end 74.295 73.1697) (width 0.25) (layer B.Cu) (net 10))
 (segment (start 30.48 68.58) (end 27.94 71.12) (width 0.25) (layer B.Cu) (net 10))
 (segment (start 27.94 71.12) (end 27.94 75.565) (width 0.25) (layer B.Cu) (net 10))
 (segment (start 74.155 62.4) (end 73.0297 62.4) (width 0.25) (layer F.Cu) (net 10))
 (segment (start 73.0297 62.4) (end 71.7166 61.0869) (width 0.25) (layer F.Cu) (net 10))
 (segment (start 71.7166 61.0869) (end 37.9731 61.0869) (width 0.25) (layer F.Cu) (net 10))
 (segment (start 37.9731 61.0869) (end 30.48 68.58) (width 0.25) (layer F.Cu) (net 10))
 (segment (start 59.275 81.85) (end 60.4654 83.0404) (width 0.25) (layer B.Cu) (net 11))
 (segment (start 60.4654 83.0404) (end 70.3931 83.0404) (width 0.25) (layer B.Cu) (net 11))
 (segment (start 70.3931 83.0404) (end 79.7735 73.66) (width 0.25) (layer B.Cu) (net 11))
 (segment (start 79.7735 73.66) (end 81.28 73.66) (width 0.25) (layer B.Cu) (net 11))
 (segment (start 29.1153 78.105) (end 30.2906 79.2803) (width 0.25) (layer F.Cu) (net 11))
 (segment (start 30.2906 79.2803) (end 44.1803 79.2803) (width 0.25) (layer F.Cu) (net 11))
 (segment (start 44.1803 79.2803) (end 48.4431 83.5431) (width 0.25) (layer F.Cu) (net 11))
 (segment (start 48.4431 83.5431) (end 57.5819 83.5431) (width 0.25) (layer F.Cu) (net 11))
 (segment (start 57.5819 83.5431) (end 59.275 81.85) (width 0.25) (layer F.Cu) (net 11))
 (segment (start 27.94 78.105) (end 29.1153 78.105) (width 0.25) (layer F.Cu) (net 11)))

